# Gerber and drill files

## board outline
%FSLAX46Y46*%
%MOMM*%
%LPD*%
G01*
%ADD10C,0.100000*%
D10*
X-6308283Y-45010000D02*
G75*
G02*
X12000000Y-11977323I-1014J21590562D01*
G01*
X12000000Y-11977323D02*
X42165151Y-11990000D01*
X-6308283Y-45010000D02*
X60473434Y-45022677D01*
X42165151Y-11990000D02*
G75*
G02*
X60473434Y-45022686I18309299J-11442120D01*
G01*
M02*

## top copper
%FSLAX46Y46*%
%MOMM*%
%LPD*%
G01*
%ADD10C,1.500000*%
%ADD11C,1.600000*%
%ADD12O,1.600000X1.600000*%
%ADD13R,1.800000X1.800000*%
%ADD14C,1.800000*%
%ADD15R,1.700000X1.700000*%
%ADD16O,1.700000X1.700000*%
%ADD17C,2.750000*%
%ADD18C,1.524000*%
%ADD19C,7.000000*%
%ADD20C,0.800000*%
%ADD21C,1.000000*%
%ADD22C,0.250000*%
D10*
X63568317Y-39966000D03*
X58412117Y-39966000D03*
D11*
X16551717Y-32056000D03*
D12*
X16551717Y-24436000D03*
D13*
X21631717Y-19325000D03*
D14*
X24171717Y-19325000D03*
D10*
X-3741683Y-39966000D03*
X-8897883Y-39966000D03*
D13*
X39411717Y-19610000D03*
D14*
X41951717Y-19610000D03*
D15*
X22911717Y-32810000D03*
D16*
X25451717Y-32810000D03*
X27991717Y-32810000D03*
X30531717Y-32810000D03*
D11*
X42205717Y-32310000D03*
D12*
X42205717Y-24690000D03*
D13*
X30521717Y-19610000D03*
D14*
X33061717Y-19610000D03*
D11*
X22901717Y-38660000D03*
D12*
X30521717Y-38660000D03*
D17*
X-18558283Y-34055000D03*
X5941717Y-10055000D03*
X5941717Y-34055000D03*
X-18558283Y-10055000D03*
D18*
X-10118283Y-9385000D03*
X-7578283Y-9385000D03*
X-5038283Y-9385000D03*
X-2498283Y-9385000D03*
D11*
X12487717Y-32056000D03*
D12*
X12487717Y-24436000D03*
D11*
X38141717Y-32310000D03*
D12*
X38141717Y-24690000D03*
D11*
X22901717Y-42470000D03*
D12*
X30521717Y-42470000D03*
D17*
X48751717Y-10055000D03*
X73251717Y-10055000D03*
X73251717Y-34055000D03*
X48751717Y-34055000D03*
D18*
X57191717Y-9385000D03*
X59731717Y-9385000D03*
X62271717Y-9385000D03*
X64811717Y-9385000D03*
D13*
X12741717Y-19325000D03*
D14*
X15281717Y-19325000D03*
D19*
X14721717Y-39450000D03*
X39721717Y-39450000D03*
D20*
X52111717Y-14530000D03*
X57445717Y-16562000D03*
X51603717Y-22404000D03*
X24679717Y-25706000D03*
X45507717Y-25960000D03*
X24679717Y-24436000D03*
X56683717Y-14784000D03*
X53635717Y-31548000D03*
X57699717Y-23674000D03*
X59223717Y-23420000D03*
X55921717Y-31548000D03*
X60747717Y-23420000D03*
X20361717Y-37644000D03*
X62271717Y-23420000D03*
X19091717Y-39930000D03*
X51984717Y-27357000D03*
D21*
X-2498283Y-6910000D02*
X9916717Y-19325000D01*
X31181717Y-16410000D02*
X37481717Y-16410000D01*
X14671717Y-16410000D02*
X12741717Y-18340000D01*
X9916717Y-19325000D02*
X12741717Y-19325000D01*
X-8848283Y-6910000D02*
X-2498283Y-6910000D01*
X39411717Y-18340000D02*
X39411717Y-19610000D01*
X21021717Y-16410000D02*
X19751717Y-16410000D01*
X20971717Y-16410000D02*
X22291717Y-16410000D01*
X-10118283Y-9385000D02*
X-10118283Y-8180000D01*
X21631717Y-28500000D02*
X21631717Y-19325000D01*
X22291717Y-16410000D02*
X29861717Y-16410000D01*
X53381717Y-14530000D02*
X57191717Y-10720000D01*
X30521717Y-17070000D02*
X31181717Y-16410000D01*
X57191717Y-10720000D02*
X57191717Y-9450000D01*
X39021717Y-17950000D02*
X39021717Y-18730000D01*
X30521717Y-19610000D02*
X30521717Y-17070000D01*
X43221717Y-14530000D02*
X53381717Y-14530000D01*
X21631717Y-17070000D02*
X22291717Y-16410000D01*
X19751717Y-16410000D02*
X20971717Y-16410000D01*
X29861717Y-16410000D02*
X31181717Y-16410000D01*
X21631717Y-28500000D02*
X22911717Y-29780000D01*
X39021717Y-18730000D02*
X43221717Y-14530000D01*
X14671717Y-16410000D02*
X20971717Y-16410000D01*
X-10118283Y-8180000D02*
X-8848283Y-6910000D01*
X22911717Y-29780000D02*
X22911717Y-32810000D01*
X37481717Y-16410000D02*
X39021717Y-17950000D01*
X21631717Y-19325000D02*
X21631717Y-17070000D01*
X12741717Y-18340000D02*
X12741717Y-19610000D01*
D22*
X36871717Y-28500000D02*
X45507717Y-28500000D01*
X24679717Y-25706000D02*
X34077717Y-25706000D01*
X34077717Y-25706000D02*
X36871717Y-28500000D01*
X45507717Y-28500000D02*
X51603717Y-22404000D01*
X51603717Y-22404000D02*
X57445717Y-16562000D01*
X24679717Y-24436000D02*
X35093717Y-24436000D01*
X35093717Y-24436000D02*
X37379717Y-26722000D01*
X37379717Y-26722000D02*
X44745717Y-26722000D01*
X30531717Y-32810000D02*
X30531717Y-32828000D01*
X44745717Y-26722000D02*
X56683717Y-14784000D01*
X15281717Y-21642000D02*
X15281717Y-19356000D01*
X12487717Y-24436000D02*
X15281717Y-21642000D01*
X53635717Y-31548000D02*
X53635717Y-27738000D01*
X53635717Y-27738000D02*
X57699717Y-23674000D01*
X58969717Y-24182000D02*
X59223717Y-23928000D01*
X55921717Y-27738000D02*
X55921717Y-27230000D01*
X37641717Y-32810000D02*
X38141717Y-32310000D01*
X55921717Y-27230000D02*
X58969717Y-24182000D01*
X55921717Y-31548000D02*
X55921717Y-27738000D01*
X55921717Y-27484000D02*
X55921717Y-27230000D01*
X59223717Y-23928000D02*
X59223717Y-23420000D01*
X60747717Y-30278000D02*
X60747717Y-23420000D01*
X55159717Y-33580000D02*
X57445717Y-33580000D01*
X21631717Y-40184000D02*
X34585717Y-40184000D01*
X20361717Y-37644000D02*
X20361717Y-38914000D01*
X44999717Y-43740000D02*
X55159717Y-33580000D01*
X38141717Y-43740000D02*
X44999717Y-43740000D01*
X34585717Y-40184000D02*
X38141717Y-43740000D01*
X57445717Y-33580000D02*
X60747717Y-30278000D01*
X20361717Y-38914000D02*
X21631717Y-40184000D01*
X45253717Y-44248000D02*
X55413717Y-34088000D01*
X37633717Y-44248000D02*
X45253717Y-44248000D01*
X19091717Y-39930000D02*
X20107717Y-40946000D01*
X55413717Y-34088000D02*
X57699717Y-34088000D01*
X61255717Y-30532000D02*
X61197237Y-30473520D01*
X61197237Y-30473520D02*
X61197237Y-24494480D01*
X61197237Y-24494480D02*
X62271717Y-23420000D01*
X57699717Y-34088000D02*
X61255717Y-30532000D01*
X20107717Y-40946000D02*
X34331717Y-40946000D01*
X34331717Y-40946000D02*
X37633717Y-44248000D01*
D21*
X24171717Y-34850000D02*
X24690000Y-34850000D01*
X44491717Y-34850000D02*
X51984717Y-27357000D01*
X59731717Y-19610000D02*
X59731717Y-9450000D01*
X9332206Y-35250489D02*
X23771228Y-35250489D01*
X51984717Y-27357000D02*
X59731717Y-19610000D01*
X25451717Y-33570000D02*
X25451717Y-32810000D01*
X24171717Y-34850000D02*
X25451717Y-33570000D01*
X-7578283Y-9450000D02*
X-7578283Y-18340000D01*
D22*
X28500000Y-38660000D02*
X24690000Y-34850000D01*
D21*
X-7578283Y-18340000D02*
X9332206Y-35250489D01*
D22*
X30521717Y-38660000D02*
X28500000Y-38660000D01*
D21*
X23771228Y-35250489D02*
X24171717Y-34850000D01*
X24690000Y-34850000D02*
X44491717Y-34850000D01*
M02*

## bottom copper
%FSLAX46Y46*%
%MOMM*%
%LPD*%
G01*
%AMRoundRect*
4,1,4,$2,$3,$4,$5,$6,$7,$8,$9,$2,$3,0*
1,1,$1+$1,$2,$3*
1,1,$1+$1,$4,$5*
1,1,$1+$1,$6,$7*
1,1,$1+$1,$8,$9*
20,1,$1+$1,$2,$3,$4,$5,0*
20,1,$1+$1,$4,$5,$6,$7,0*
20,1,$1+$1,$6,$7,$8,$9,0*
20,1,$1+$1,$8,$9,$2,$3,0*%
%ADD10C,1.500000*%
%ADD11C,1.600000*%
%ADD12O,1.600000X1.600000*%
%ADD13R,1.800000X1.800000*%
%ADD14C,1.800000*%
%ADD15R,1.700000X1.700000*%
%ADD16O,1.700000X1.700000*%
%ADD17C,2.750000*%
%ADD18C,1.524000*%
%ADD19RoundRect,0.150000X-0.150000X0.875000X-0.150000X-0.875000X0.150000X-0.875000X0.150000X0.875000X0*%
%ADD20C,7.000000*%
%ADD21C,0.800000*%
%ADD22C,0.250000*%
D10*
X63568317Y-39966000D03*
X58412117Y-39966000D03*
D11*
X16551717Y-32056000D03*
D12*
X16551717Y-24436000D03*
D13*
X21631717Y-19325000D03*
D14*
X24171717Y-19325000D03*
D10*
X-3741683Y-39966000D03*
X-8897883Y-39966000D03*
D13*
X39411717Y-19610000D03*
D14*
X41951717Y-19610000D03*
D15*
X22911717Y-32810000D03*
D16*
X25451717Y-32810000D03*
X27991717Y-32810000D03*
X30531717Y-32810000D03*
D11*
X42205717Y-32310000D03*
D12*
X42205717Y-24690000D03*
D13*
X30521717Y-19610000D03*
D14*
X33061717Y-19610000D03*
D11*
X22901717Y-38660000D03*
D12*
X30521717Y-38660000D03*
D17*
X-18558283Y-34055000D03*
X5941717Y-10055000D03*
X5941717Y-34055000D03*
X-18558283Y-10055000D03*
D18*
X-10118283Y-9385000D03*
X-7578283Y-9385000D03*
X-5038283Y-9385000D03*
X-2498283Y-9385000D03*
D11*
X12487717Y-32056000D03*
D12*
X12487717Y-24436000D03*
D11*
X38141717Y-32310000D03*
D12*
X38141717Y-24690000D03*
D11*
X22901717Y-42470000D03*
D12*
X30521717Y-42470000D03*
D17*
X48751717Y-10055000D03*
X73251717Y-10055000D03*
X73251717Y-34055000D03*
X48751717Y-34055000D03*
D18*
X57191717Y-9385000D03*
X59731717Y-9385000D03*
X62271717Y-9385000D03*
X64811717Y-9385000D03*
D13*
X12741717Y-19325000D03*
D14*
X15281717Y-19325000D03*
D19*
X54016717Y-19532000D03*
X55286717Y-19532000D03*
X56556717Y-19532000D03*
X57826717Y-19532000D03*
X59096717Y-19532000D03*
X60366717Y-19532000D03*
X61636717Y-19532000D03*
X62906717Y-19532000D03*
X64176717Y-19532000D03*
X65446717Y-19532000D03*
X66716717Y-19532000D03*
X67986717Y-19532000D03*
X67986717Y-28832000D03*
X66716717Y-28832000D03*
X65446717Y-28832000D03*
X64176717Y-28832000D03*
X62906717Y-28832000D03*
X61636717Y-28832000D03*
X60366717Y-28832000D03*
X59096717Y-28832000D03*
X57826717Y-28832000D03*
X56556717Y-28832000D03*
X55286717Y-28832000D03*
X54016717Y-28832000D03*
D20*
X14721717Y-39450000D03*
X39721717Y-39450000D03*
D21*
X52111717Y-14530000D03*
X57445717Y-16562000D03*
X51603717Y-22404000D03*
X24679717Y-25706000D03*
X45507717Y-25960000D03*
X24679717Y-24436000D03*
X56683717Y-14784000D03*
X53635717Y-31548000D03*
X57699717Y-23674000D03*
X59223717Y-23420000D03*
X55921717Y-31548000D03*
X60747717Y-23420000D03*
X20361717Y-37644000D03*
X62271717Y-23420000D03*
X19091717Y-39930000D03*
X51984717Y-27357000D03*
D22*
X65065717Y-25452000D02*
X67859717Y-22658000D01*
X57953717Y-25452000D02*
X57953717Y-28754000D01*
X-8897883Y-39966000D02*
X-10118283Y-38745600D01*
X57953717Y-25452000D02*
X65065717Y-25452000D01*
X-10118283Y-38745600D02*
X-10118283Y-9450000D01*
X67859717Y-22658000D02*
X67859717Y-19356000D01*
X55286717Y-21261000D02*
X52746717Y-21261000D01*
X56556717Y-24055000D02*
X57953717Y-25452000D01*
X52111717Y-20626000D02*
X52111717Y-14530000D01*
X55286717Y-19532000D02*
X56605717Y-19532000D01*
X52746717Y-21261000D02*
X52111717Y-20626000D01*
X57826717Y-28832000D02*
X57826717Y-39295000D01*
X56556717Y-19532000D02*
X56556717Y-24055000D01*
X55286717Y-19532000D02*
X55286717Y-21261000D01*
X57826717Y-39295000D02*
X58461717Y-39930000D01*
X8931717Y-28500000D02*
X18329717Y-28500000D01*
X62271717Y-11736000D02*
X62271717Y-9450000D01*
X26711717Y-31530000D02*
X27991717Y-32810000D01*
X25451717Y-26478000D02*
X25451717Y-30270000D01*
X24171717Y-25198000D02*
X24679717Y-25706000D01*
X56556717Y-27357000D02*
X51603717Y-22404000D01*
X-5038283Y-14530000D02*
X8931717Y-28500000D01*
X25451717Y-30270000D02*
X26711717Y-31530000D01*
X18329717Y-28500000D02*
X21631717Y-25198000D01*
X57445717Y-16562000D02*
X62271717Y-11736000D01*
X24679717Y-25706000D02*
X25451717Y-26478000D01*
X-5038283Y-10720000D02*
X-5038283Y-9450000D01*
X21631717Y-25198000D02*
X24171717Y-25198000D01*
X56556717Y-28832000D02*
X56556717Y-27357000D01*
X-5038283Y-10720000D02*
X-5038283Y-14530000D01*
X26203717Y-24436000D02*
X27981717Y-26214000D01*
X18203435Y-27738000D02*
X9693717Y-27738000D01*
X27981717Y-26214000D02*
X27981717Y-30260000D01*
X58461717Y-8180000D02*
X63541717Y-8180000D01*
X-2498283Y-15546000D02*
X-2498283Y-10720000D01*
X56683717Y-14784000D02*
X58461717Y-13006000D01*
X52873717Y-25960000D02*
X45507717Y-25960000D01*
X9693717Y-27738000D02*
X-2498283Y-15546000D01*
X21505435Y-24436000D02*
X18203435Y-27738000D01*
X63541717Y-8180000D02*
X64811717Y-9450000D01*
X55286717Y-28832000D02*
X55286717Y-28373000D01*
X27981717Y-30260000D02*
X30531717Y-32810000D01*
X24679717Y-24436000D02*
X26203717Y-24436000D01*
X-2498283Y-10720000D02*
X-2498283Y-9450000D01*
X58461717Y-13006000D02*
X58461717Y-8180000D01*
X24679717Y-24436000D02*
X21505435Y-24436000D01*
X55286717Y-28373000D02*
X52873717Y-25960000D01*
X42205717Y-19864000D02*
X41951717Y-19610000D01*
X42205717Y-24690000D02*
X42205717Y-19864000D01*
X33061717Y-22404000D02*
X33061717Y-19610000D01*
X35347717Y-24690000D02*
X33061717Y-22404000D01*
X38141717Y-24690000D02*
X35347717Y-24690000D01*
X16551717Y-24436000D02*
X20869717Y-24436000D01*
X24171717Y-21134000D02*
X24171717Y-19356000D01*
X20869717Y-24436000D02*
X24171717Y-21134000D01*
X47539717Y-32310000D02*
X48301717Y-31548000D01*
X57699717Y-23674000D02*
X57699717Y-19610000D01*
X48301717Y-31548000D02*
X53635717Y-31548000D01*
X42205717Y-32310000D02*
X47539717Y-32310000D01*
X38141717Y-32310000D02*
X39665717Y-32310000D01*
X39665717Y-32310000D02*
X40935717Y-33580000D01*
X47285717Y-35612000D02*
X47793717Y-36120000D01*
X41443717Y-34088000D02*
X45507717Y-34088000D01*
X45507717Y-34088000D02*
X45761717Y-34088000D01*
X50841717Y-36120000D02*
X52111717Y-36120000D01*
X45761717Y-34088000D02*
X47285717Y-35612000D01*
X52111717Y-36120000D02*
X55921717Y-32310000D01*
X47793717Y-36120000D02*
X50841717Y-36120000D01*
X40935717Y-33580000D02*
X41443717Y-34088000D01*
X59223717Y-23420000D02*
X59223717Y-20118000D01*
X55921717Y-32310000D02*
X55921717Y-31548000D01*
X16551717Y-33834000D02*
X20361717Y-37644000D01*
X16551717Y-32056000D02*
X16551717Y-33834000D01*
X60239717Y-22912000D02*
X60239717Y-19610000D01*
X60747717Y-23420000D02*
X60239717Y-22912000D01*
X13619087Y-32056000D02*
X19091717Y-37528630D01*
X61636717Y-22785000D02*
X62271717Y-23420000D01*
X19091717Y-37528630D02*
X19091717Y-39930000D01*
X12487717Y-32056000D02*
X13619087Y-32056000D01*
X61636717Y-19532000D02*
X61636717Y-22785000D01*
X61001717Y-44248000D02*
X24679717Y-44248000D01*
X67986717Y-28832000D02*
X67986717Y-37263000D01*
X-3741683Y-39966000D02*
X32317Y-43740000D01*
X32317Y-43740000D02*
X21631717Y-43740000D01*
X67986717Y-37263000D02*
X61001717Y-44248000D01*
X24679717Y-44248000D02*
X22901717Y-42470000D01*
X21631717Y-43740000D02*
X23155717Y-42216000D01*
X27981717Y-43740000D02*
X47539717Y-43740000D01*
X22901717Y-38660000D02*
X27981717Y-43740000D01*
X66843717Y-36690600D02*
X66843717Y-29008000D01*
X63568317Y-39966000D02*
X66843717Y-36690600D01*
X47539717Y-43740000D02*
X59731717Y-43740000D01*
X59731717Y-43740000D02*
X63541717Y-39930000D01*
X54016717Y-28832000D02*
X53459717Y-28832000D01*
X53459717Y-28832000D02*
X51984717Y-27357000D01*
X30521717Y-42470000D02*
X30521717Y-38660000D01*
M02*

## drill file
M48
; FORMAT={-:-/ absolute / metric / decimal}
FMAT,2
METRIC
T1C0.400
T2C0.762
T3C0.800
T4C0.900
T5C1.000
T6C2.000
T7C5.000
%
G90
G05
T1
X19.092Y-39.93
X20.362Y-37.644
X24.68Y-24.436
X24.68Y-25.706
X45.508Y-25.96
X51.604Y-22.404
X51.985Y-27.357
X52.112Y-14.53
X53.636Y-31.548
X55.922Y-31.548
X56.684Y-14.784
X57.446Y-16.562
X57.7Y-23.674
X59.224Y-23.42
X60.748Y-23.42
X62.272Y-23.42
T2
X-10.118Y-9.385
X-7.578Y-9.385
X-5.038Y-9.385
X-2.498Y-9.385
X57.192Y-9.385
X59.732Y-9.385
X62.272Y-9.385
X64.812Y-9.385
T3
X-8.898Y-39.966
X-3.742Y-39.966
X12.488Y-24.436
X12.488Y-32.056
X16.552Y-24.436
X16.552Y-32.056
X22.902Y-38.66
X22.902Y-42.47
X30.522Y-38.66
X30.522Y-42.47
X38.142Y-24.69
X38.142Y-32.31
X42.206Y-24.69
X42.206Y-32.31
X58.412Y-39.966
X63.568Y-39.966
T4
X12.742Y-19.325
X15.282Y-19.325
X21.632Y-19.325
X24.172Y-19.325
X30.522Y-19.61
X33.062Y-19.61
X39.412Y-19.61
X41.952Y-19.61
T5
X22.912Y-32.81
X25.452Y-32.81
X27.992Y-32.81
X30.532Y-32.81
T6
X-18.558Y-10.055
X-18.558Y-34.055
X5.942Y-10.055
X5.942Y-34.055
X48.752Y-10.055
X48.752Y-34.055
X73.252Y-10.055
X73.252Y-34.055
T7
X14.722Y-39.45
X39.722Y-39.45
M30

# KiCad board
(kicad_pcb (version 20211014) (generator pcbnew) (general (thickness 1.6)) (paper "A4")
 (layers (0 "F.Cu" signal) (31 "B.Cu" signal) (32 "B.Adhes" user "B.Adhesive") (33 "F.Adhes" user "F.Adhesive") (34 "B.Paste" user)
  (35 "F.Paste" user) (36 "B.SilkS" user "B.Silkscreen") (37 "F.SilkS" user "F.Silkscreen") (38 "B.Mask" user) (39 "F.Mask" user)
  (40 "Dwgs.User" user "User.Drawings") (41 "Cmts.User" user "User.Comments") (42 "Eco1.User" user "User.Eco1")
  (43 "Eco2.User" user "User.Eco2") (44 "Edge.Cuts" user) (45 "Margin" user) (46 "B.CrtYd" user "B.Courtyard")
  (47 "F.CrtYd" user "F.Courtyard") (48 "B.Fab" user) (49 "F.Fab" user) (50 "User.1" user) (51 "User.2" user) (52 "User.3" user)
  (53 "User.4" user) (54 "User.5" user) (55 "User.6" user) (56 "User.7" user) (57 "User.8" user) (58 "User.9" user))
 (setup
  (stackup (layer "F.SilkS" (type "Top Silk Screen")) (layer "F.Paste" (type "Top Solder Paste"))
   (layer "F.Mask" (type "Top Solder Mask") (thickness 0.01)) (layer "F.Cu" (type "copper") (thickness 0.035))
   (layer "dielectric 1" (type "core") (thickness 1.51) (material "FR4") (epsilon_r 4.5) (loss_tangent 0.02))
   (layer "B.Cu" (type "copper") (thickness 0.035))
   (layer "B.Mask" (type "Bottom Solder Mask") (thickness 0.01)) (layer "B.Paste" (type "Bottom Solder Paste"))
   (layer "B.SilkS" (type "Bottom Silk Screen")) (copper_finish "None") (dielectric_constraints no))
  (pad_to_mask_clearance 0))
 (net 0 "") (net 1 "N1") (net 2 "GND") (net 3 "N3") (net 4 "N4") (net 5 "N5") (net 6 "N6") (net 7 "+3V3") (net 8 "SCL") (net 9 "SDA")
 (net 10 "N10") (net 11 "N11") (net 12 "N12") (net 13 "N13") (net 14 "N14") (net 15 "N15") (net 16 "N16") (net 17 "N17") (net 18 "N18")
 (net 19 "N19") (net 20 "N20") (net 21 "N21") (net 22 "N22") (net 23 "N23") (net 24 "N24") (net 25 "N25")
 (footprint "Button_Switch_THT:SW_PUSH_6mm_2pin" (layer "F.Cu") (at 57.751717 37.68)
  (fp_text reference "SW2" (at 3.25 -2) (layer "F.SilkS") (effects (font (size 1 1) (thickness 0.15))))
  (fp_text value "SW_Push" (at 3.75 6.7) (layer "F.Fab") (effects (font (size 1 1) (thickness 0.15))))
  (pad "1" thru_hole circle (at 5.8166 2.286 90) (size 1.5 1.5) (drill 0.8) (layers *.Cu *.Mask) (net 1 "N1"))
  (pad "2" thru_hole circle (at 0.6604 2.286 90) (size 1.5 1.5) (drill 0.8) (layers *.Cu *.Mask) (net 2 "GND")))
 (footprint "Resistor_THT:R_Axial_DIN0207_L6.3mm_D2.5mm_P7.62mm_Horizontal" (layer "F.Cu") (at 16.551717 32.056 90)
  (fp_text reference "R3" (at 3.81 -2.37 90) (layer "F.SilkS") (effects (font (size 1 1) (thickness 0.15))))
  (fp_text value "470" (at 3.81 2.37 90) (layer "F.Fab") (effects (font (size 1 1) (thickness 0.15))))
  (pad "1" thru_hole circle (at 0 0 90) (size 1.6 1.6) (drill 0.8) (layers *.Cu *.Mask) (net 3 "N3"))
  (pad "2" thru_hole oval (at 7.62 0 90) (size 1.6 1.6) (drill 0.8) (layers *.Cu *.Mask) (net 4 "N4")))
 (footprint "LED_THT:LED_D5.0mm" (layer "F.Cu") (at 21.631717 19.325)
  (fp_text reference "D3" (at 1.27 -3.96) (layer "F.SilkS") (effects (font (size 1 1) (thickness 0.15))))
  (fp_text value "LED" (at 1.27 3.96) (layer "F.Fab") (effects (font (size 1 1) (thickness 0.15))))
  (pad "1" thru_hole rect (at 0 0) (size 1.8 1.8) (drill 0.9) (layers *.Cu *.Mask) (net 2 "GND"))
  (pad "2" thru_hole circle (at 2.54 0) (size 1.8 1.8) (drill 0.9) (layers *.Cu *.Mask) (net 4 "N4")))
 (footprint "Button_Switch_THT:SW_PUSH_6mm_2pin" (layer "F.Cu") (at -9.558283 37.68)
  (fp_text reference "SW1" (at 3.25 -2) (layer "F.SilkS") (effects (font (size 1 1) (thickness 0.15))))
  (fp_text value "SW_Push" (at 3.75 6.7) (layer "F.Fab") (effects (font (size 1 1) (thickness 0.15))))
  (pad "1" thru_hole circle (at 5.8166 2.286 90) (size 1.5 1.5) (drill 0.8) (layers *.Cu *.Mask) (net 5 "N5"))
  (pad "2" thru_hole circle (at 0.6604 2.286 90) (size 1.5 1.5) (drill 0.8) (layers *.Cu *.Mask) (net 2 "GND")))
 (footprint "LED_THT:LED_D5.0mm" (layer "F.Cu") (at 39.411717 19.61)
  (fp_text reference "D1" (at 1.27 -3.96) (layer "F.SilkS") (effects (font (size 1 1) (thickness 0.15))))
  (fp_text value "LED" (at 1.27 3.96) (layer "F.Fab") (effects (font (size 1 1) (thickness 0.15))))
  (pad "1" thru_hole rect (at 0 0) (size 1.8 1.8) (drill 0.9) (layers *.Cu *.Mask) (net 2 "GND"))
  (pad "2" thru_hole circle (at 2.54 0) (size 1.8 1.8) (drill 0.9) (layers *.Cu *.Mask) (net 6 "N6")))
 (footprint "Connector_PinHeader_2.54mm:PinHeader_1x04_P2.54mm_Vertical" (layer "F.Cu") (at 22.911717 32.81 90)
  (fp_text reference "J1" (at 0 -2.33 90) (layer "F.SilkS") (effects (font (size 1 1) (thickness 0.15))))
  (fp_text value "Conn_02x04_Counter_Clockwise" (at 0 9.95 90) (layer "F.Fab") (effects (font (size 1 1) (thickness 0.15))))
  (pad "1" thru_hole rect (at 0 0 90) (size 1.7 1.7) (drill 1) (layers *.Cu *.Mask) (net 2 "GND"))
  (pad "2" thru_hole oval (at 0 2.54 90) (size 1.7 1.7) (drill 1) (layers *.Cu *.Mask) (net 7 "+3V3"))
  (pad "3" thru_hole oval (at 0 5.08 90) (size 1.7 1.7) (drill 1) (layers *.Cu *.Mask) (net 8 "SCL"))
  (pad "4" thru_hole oval (at 0 7.62 90) (size 1.7 1.7) (drill 1) (layers *.Cu *.Mask) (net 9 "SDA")))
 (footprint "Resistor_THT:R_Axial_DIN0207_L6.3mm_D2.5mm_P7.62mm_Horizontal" (layer "F.Cu") (at 42.205717 32.31 90)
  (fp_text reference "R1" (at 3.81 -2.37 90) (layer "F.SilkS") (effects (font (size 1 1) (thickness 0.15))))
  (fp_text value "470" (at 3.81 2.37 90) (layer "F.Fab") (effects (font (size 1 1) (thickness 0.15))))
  (pad "1" thru_hole circle (at 0 0 90) (size 1.6 1.6) (drill 0.8) (layers *.Cu *.Mask) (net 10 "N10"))
  (pad "2" thru_hole oval (at 7.62 0 90) (size 1.6 1.6) (drill 0.8) (layers *.Cu *.Mask) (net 6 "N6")))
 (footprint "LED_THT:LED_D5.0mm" (layer "F.Cu") (at 30.521717 19.61)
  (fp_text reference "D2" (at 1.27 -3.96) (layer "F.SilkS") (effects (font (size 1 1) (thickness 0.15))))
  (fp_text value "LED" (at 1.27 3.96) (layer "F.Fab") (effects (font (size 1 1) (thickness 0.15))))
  (pad "1" thru_hole rect (at 0 0) (size 1.8 1.8) (drill 0.9) (layers *.Cu *.Mask) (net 2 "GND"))
  (pad "2" thru_hole circle (at 2.54 0) (size 1.8 1.8) (drill 0.9) (layers *.Cu *.Mask) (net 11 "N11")))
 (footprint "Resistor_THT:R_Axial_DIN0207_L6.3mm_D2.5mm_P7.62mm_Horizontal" (layer "F.Cu") (at 22.901717 38.66)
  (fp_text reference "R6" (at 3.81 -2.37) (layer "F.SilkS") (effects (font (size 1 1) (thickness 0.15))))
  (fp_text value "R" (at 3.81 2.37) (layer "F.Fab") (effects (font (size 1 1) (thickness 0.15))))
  (pad "1" thru_hole circle (at 0 0) (size 1.6 1.6) (drill 0.8) (layers *.Cu *.Mask) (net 1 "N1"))
  (pad "2" thru_hole oval (at 7.62 0) (size 1.6 1.6) (drill 0.8) (layers *.Cu *.Mask) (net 7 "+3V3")))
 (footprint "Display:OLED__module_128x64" (layer "F.Cu") (at -6.308283 36.055)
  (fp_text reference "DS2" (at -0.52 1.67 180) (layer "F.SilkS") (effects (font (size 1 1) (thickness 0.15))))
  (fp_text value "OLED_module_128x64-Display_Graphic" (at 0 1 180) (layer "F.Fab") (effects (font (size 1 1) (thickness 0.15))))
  (pad "" thru_hole circle (at -12.25 -2) (size 2.75 2.75) (drill 2) (layers *.Cu *.Mask))
  (pad "" thru_hole circle (at 12.25 -26) (size 2.75 2.75) (drill 2) (layers *.Cu *.Mask))
  (pad "" thru_hole circle (at 12.25 -2) (size 2.75 2.75) (drill 2) (layers *.Cu *.Mask))
  (pad "" thru_hole circle (at -12.25 -26) (size 2.75 2.75) (drill 2) (layers *.Cu *.Mask))
  (pad "1" thru_hole circle (at -3.81 -26.67) (size 1.524 1.524) (drill 0.762) (layers *.Cu *.Mask) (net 2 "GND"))
  (pad "2" thru_hole circle (at -1.27 -26.67) (size 1.524 1.524) (drill 0.762) (layers *.Cu *.Mask) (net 7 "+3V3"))
  (pad "3" thru_hole circle (at 1.27 -26.67) (size 1.524 1.524) (drill 0.762) (layers *.Cu *.Mask) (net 8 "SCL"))
  (pad "4" thru_hole circle (at 3.81 -26.67) (size 1.524 1.524) (drill 0.762) (layers *.Cu *.Mask) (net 9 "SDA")))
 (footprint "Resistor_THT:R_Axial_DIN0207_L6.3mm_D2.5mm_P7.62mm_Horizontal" (layer "F.Cu") (at 12.487717 32.056 90)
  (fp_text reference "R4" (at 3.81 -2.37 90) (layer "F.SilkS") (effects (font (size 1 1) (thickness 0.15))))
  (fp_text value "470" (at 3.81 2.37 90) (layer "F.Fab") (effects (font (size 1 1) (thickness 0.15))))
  (pad "1" thru_hole circle (at 0 0 90) (size 1.6 1.6) (drill 0.8) (layers *.Cu *.Mask) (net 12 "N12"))
  (pad "2" thru_hole oval (at 7.62 0 90) (size 1.6 1.6) (drill 0.8) (layers *.Cu *.Mask) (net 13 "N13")))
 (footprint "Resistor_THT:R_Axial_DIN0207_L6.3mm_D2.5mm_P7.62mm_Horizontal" (layer "F.Cu") (at 38.141717 32.31 90)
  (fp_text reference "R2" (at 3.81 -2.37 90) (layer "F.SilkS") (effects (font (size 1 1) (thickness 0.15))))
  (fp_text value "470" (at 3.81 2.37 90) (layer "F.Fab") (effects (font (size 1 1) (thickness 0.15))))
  (pad "1" thru_hole circle (at 0 0 90) (size 1.6 1.6) (drill 0.8) (layers *.Cu *.Mask) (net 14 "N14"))
  (pad "2" thru_hole oval (at 7.62 0 90) (size 1.6 1.6) (drill 0.8) (layers *.Cu *.Mask) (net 11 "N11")))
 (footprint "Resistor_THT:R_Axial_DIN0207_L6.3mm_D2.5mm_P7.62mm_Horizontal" (layer "F.Cu") (at 22.901717 42.47)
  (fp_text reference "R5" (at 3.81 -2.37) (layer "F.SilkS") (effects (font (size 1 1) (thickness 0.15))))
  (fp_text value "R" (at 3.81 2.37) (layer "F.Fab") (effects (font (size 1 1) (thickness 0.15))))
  (pad "1" thru_hole circle (at 0 0) (size 1.6 1.6) (drill 0.8) (layers *.Cu *.Mask) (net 5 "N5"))
  (pad "2" thru_hole oval (at 7.62 0) (size 1.6 1.6) (drill 0.8) (layers *.Cu *.Mask) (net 7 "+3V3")))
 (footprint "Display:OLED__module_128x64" (layer "F.Cu") (at 61.001717 36.055)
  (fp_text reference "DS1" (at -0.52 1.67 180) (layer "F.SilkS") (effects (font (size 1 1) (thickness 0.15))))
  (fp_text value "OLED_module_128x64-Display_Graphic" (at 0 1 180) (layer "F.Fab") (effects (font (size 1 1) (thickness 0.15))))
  (pad "" thru_hole circle (at -12.25 -26) (size 2.75 2.75) (drill 2) (layers *.Cu *.Mask))
  (pad "" thru_hole circle (at 12.25 -26) (size 2.75 2.75) (drill 2) (layers *.Cu *.Mask))
  (pad "" thru_hole circle (at 12.25 -2) (size 2.75 2.75) (drill 2) (layers *.Cu *.Mask))
  (pad "" thru_hole circle (at -12.25 -2) (size 2.75 2.75) (drill 2) (layers *.Cu *.Mask))
  (pad "1" thru_hole circle (at -3.81 -26.67) (size 1.524 1.524) (drill 0.762) (layers *.Cu *.Mask) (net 2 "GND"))
  (pad "2" thru_hole circle (at -1.27 -26.67) (size 1.524 1.524) (drill 0.762) (layers *.Cu *.Mask) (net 7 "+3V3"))
  (pad "3" thru_hole circle (at 1.27 -26.67) (size 1.524 1.524) (drill 0.762) (layers *.Cu *.Mask) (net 8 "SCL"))
  (pad "4" thru_hole circle (at 3.81 -26.67) (size 1.524 1.524) (drill 0.762) (layers *.Cu *.Mask) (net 9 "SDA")))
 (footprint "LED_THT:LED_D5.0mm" (layer "F.Cu") (at 12.741717 19.325)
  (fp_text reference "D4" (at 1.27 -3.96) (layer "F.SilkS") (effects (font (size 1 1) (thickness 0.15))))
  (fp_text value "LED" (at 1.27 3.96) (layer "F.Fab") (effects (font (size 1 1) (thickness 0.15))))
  (pad "1" thru_hole rect (at 0 0) (size 1.8 1.8) (drill 0.9) (layers *.Cu *.Mask) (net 2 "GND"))
  (pad "2" thru_hole circle (at 2.54 0) (size 1.8 1.8) (drill 0.9) (layers *.Cu *.Mask) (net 13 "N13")))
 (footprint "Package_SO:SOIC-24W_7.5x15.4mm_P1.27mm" (layer "B.Cu") (at 61.001717 24.182 -90)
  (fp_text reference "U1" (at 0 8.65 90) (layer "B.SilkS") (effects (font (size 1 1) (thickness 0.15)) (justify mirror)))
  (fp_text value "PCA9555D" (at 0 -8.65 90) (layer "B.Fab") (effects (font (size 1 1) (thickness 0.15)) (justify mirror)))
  (pad "1" smd roundrect (at -4.65 6.985 270) (size 2.05 0.6) (layers "B.Cu" "B.Paste" "B.Mask") (roundrect_rratio 0.25) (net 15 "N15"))
  (pad "2" smd roundrect (at -4.65 5.715 270) (size 2.05 0.6) (layers "B.Cu" "B.Paste" "B.Mask") (roundrect_rratio 0.25) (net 2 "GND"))
  (pad "3" smd roundrect (at -4.65 4.445 270) (size 2.05 0.6) (layers "B.Cu" "B.Paste" "B.Mask") (roundrect_rratio 0.25) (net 2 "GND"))
  (pad "4" smd roundrect (at -4.65 3.175 270) (size 2.05 0.6) (layers "B.Cu" "B.Paste" "B.Mask") (roundrect_rratio 0.25) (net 10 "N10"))
  (pad "5" smd roundrect (at -4.65 1.905 270) (size 2.05 0.6) (layers "B.Cu" "B.Paste" "B.Mask") (roundrect_rratio 0.25) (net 14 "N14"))
  (pad "6" smd roundrect (at -4.65 0.635 270) (size 2.05 0.6) (layers "B.Cu" "B.Paste" "B.Mask") (roundrect_rratio 0.25) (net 3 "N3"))
  (pad "7" smd roundrect (at -4.65 -0.635 270) (size 2.05 0.6) (layers "B.Cu" "B.Paste" "B.Mask") (roundrect_rratio 0.25) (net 12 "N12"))
  (pad "8" smd roundrect (at -4.65 -1.905 270) (size 2.05 0.6) (layers "B.Cu" "B.Paste" "B.Mask") (roundrect_rratio 0.25) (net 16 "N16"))
  (pad "9" smd roundrect (at -4.65 -3.175 270) (size 2.05 0.6) (layers "B.Cu" "B.Paste" "B.Mask") (roundrect_rratio 0.25) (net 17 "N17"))
  (pad "10" smd roundrect (at -4.65 -4.445 270) (size 2.05 0.6) (layers "B.Cu" "B.Paste" "B.Mask") (roundrect_rratio 0.25) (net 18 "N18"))
  (pad "11" smd roundrect (at -4.65 -5.715 270) (size 2.05 0.6) (layers "B.Cu" "B.Paste" "B.Mask") (roundrect_rratio 0.25) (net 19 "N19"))
  (pad "12" smd roundrect (at -4.65 -6.985 270) (size 2.05 0.6) (layers "B.Cu" "B.Paste" "B.Mask") (roundrect_rratio 0.25) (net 2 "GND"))
  (pad "13" smd roundrect (at 4.65 -6.985 270) (size 2.05 0.6) (layers "B.Cu" "B.Paste" "B.Mask") (roundrect_rratio 0.25) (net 5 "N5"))
  (pad "14" smd roundrect (at 4.65 -5.715 270) (size 2.05 0.6) (layers "B.Cu" "B.Paste" "B.Mask") (roundrect_rratio 0.25) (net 1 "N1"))
  (pad "15" smd roundrect (at 4.65 -4.445 270) (size 2.05 0.6) (layers "B.Cu" "B.Paste" "B.Mask") (roundrect_rratio 0.25) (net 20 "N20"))
  (pad "16" smd roundrect (at 4.65 -3.175 270) (size 2.05 0.6) (layers "B.Cu" "B.Paste" "B.Mask") (roundrect_rratio 0.25) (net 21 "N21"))
  (pad "17" smd roundrect (at 4.65 -1.905 270) (size 2.05 0.6) (layers "B.Cu" "B.Paste" "B.Mask") (roundrect_rratio 0.25) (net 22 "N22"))
  (pad "18" smd roundrect (at 4.65 -0.635 270) (size 2.05 0.6) (layers "B.Cu" "B.Paste" "B.Mask") (roundrect_rratio 0.25) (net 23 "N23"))
  (pad "19" smd roundrect (at 4.65 0.635 270) (size 2.05 0.6) (layers "B.Cu" "B.Paste" "B.Mask") (roundrect_rratio 0.25) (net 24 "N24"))
  (pad "20" smd roundrect (at 4.65 1.905 270) (size 2.05 0.6) (layers "B.Cu" "B.Paste" "B.Mask") (roundrect_rratio 0.25) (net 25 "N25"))
  (pad "21" smd roundrect (at 4.65 3.175 270) (size 2.05 0.6) (layers "B.Cu" "B.Paste" "B.Mask") (roundrect_rratio 0.25) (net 2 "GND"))
  (pad "22" smd roundrect (at 4.65 4.445 270) (size 2.05 0.6) (layers "B.Cu" "B.Paste" "B.Mask") (roundrect_rratio 0.25) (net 8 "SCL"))
  (pad "23" smd roundrect (at 4.65 5.715 270) (size 2.05 0.6) (layers "B.Cu" "B.Paste" "B.Mask") (roundrect_rratio 0.25) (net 9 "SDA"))
  (pad "24" smd roundrect (at 4.65 6.985 270) (size 2.05 0.6) (layers "B.Cu" "B.Paste" "B.Mask") (roundrect_rratio 0.25) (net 7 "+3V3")))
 (gr_arc (start -6.308283 45.01) (mid -25.19332 12.953013) (end 12 11.977323) (layer "Edge.Cuts") (width 0.1))
 (gr_line (start 12 11.977323) (end 42.165151 11.99) (layer "Edge.Cuts") (width 0.1))
 (gr_line (start -6.308283 45.01) (end 60.473434 45.022677) (layer "Edge.Cuts") (width 0.1))
 (gr_arc (start 42.165151 11.99) (mid 79.35847 12.96569) (end 60.473434 45.022677) (layer "Edge.Cuts") (width 0.1))
 (via (at 14.721717 39.45) (size 7) (drill 5) (layers "F.Cu" "B.Cu") (free) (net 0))
 (via (at 39.721717 39.45) (size 7) (drill 5) (layers "F.Cu" "B.Cu") (free) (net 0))
 (segment (start -2.498283 6.91) (end 9.916717 19.325) (width 1) (layer "F.Cu") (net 2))
 (segment (start 31.181717 16.41) (end 37.481717 16.41) (width 1) (layer "F.Cu") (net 2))
 (segment (start 14.671717 16.41) (end 12.741717 18.34) (width 1) (layer "F.Cu") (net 2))
 (segment (start 9.916717 19.325) (end 12.741717 19.325) (width 1) (layer "F.Cu") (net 2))
 (segment (start -8.848283 6.91) (end -2.498283 6.91) (width 1) (layer "F.Cu") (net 2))
 (segment (start 39.411717 18.34) (end 39.411717 19.61) (width 1) (layer "F.Cu") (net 2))
 (segment (start 21.021717 16.41) (end 19.751717 16.41) (width 1) (layer "F.Cu") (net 2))
 (segment (start 20.971717 16.41) (end 22.291717 16.41) (width 1) (layer "F.Cu") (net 2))
 (segment (start -10.118283 9.385) (end -10.118283 8.18) (width 1) (layer "F.Cu") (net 2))
 (segment (start 21.631717 28.5) (end 21.631717 19.325) (width 1) (layer "F.Cu") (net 2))
 (segment (start 22.291717 16.41) (end 29.861717 16.41) (width 1) (layer "F.Cu") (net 2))
 (segment (start 53.381717 14.53) (end 57.191717 10.72) (width 1) (layer "F.Cu") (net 2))
 (segment (start 30.521717 17.07) (end 31.181717 16.41) (width 1) (layer "F.Cu") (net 2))
 (segment (start 57.191717 10.72) (end 57.191717 9.45) (width 1) (layer "F.Cu") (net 2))
 (segment (start 39.021717 17.95) (end 39.021717 18.73) (width 1) (layer "F.Cu") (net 2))
 (segment (start 30.521717 19.61) (end 30.521717 17.07) (width 1) (layer "F.Cu") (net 2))
 (segment (start 43.221717 14.53) (end 53.381717 14.53) (width 1) (layer "F.Cu") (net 2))
 (segment (start 21.631717 17.07) (end 22.291717 16.41) (width 1) (layer "F.Cu") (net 2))
 (segment (start 19.751717 16.41) (end 20.971717 16.41) (width 1) (layer "F.Cu") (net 2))
 (segment (start 29.861717 16.41) (end 31.181717 16.41) (width 1) (layer "F.Cu") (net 2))
 (segment (start 21.631717 28.5) (end 22.911717 29.78) (width 1) (layer "F.Cu") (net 2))
 (segment (start 39.021717 18.73) (end 43.221717 14.53) (width 1) (layer "F.Cu") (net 2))
 (segment (start 14.671717 16.41) (end 20.971717 16.41) (width 1) (layer "F.Cu") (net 2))
 (segment (start -10.118283 8.18) (end -8.848283 6.91) (width 1) (layer "F.Cu") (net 2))
 (segment (start 22.911717 29.78) (end 22.911717 32.81) (width 1) (layer "F.Cu") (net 2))
 (segment (start 37.481717 16.41) (end 39.021717 17.95) (width 1) (layer "F.Cu") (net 2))
 (segment (start 21.631717 19.325) (end 21.631717 17.07) (width 1) (layer "F.Cu") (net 2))
 (segment (start 12.741717 18.34) (end 12.741717 19.61) (width 1) (layer "F.Cu") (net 2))
 (via (at 52.111717 14.53) (size 0.8) (drill 0.4) (layers "F.Cu" "B.Cu") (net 2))
 (segment (start 65.065717 25.452) (end 67.859717 22.658) (width 0.25) (layer "B.Cu") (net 2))
 (segment (start 57.953717 25.452) (end 57.953717 28.754) (width 0.25) (layer "B.Cu") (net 2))
 (segment (start -8.897883 39.966) (end -10.118283 38.7456) (width 0.25) (layer "B.Cu") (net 2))
 (segment (start 57.953717 25.452) (end 65.065717 25.452) (width 0.25) (layer "B.Cu") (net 2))
 (segment (start -10.118283 38.7456) (end -10.118283 9.45) (width 0.25) (layer "B.Cu") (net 2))
 (segment (start 67.859717 22.658) (end 67.859717 19.356) (width 0.25) (layer "B.Cu") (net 2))
 (segment (start 55.286717 21.261) (end 52.746717 21.261) (width 0.25) (layer "B.Cu") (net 2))
 (segment (start 56.556717 24.055) (end 57.953717 25.452) (width 0.25) (layer "B.Cu") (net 2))
 (segment (start 52.111717 20.626) (end 52.111717 14.53) (width 0.25) (layer "B.Cu") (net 2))
 (segment (start 55.286717 19.532) (end 56.605717 19.532) (width 0.25) (layer "B.Cu") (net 2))
 (segment (start 52.746717 21.261) (end 52.111717 20.626) (width 0.25) (layer "B.Cu") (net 2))
 (segment (start 57.826717 28.832) (end 57.826717 39.295) (width 0.25) (layer "B.Cu") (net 2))
 (segment (start 56.556717 19.532) (end 56.556717 24.055) (width 0.25) (layer "B.Cu") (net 2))
 (segment (start 55.286717 19.532) (end 55.286717 21.261) (width 0.25) (layer "B.Cu") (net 2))
 (segment (start 57.826717 39.295) (end 58.461717 39.93) (width 0.25) (layer "B.Cu") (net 2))
 (segment (start 36.871717 28.5) (end 45.507717 28.5) (width 0.25) (layer "F.Cu") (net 8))
 (segment (start 24.679717 25.706) (end 34.077717 25.706) (width 0.25) (layer "F.Cu") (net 8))
 (segment (start 34.077717 25.706) (end 36.871717 28.5) (width 0.25) (layer "F.Cu") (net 8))
 (segment (start 45.507717 28.5) (end 51.603717 22.404) (width 0.25) (layer "F.Cu") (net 8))
 (segment (start 51.603717 22.404) (end 57.445717 16.562) (width 0.25) (layer "F.Cu") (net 8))
 (via (at 57.445717 16.562) (size 0.8) (drill 0.4) (layers "F.Cu" "B.Cu") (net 8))
 (via (at 51.603717 22.404) (size 0.8) (drill 0.4) (layers "F.Cu" "B.Cu") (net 8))
 (via (at 24.679717 25.706) (size 0.8) (drill 0.4) (layers "F.Cu" "B.Cu") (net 8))
 (segment (start 8.931717 28.5) (end 18.329717 28.5) (width 0.25) (layer "B.Cu") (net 8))
 (segment (start 62.271717 11.736) (end 62.271717 9.45) (width 0.25) (layer "B.Cu") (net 8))
 (segment (start 26.711717 31.53) (end 27.991717 32.81) (width 0.25) (layer "B.Cu") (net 8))
 (segment (start 25.451717 26.478) (end 25.451717 30.27) (width 0.25) (layer "B.Cu") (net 8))
 (segment (start 24.171717 25.198) (end 24.679717 25.706) (width 0.25) (layer "B.Cu") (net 8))
 (segment (start 56.556717 27.357) (end 51.603717 22.404) (width 0.25) (layer "B.Cu") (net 8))
 (segment (start -5.038283 14.53) (end 8.931717 28.5) (width 0.25) (layer "B.Cu") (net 8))
 (segment (start 25.451717 30.27) (end 26.711717 31.53) (width 0.25) (layer "B.Cu") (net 8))
 (segment (start 18.329717 28.5) (end 21.631717 25.198) (width 0.25) (layer "B.Cu") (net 8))
 (segment (start 57.445717 16.562) (end 62.271717 11.736) (width 0.25) (layer "B.Cu") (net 8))
 (segment (start 24.679717 25.706) (end 25.451717 26.478) (width 0.25) (layer "B.Cu") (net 8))
 (segment (start -5.038283 10.72) (end -5.038283 9.45) (width 0.25) (layer "B.Cu") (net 8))
 (segment (start 21.631717 25.198) (end 24.171717 25.198) (width 0.25) (layer "B.Cu") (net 8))
 (segment (start 56.556717 28.832) (end 56.556717 27.357) (width 0.25) (layer "B.Cu") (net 8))
 (segment (start -5.038283 10.72) (end -5.038283 14.53) (width 0.25) (layer "B.Cu") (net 8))
 (segment (start 24.679717 24.436) (end 35.093717 24.436) (width 0.25) (layer "F.Cu") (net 9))
 (segment (start 35.093717 24.436) (end 37.379717 26.722) (width 0.25) (layer "F.Cu") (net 9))
 (segment (start 37.379717 26.722) (end 44.745717 26.722) (width 0.25) (layer "F.Cu") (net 9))
 (segment (start 30.531717 32.81) (end 30.531717 32.828) (width 0.25) (layer "F.Cu") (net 9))
 (segment (start 44.745717 26.722) (end 56.683717 14.784) (width 0.25) (layer "F.Cu") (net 9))
 (via (at 45.507717 25.96) (size 0.8) (drill 0.4) (layers "F.Cu" "B.Cu") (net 9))
 (via (at 24.679717 24.436) (size 0.8) (drill 0.4) (layers "F.Cu" "B.Cu") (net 9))
 (via (at 56.683717 14.784) (size 0.8) (drill 0.4) (layers "F.Cu" "B.Cu") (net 9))
 (segment (start 26.203717 24.436) (end 27.981717 26.214) (width 0.25) (layer "B.Cu") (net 9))
 (segment (start 18.203435 27.738) (end 9.693717 27.738) (width 0.25) (layer "B.Cu") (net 9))
 (segment (start 27.981717 26.214) (end 27.981717 30.26) (width 0.25) (layer "B.Cu") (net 9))
 (segment (start 58.461717 8.18) (end 63.541717 8.18) (width 0.25) (layer "B.Cu") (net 9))
 (segment (start -2.498283 15.546) (end -2.498283 10.72) (width 0.25) (layer "B.Cu") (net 9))
 (segment (start 56.683717 14.784) (end 58.461717 13.006) (width 0.25) (layer "B.Cu") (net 9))
 (segment (start 52.873717 25.96) (end 45.507717 25.96) (width 0.25) (layer "B.Cu") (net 9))
 (segment (start 9.693717 27.738) (end -2.498283 15.546) (width 0.25) (layer "B.Cu") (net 9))
 (segment (start 21.505435 24.436) (end 18.203435 27.738) (width 0.25) (layer "B.Cu") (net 9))
 (segment (start 63.541717 8.18) (end 64.811717 9.45) (width 0.25) (layer "B.Cu") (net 9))
 (segment (start 55.286717 28.832) (end 55.286717 28.373) (width 0.25) (layer "B.Cu") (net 9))
 (segment (start 27.981717 30.26) (end 30.531717 32.81) (width 0.25) (layer "B.Cu") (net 9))
 (segment (start 24.679717 24.436) (end 26.203717 24.436) (width 0.25) (layer "B.Cu") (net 9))
 (segment (start -2.498283 10.72) (end -2.498283 9.45) (width 0.25) (layer "B.Cu") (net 9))
 (segment (start 58.461717 13.006) (end 58.461717 8.18) (width 0.25) (layer "B.Cu") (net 9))
 (segment (start 24.679717 24.436) (end 21.505435 24.436) (width 0.25) (layer "B.Cu") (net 9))
 (segment (start 55.286717 28.373) (end 52.873717 25.96) (width 0.25) (layer "B.Cu") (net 9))
 (segment (start 42.205717 19.864) (end 41.951717 19.61) (width 0.25) (layer "B.Cu") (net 6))
 (segment (start 42.205717 24.69) (end 42.205717 19.864) (width 0.25) (layer "B.Cu") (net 6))
 (segment (start 33.061717 22.404) (end 33.061717 19.61) (width 0.25) (layer "B.Cu") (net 11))
 (segment (start 35.347717 24.69) (end 33.061717 22.404) (width 0.25) (layer "B.Cu") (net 11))
 (segment (start 38.141717 24.69) (end 35.347717 24.69) (width 0.25) (layer "B.Cu") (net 11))
 (segment (start 16.551717 24.436) (end 20.869717 24.436) (width 0.25) (layer "B.Cu") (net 4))
 (segment (start 24.171717 21.134) (end 24.171717 19.356) (width 0.25) (layer "B.Cu") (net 4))
 (segment (start 20.869717 24.436) (end 24.171717 21.134) (width 0.25) (layer "B.Cu") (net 4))
 (segment (start 15.281717 21.642) (end 15.281717 19.356) (width 0.25) (layer "F.Cu") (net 13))
 (segment (start 12.487717 24.436) (end 15.281717 21.642) (width 0.25) (layer "F.Cu") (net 13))
 (segment (start 53.635717 31.548) (end 53.635717 27.738) (width 0.25) (layer "F.Cu") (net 10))
 (segment (start 53.635717 27.738) (end 57.699717 23.674) (width 0.25) (layer "F.Cu") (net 10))
 (via (at 53.635717 31.548) (size 0.8) (drill 0.4) (layers "F.Cu" "B.Cu") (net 10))
 (via (at 57.699717 23.674) (size 0.8) (drill 0.4) (layers "F.Cu" "B.Cu") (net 10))
 (segment (start 47.539717 32.31) (end 48.301717 31.548) (width 0.25) (layer "B.Cu") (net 10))
 (segment (start 57.699717 23.674) (end 57.699717 19.61) (width 0.25) (layer "B.Cu") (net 10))
 (segment (start 48.301717 31.548) (end 53.635717 31.548) (width 0.25) (layer "B.Cu") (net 10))
 (segment (start 42.205717 32.31) (end 47.539717 32.31) (width 0.25) (layer "B.Cu") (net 10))
 (segment (start 58.969717 24.182) (end 59.223717 23.928) (width 0.25) (layer "F.Cu") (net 14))
 (segment (start 55.921717 27.738) (end 55.921717 27.23) (width 0.25) (layer "F.Cu") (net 14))
 (segment (start 37.641717 32.81) (end 38.141717 32.31) (width 0.25) (layer "F.Cu") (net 14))
 (segment (start 55.921717 27.23) (end 58.969717 24.182) (width 0.25) (layer "F.Cu") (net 14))
 (segment (start 55.921717 31.548) (end 55.921717 27.738) (width 0.25) (layer "F.Cu") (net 14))
 (segment (start 55.921717 27.484) (end 55.921717 27.23) (width 0.25) (layer "F.Cu") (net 14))
 (segment (start 59.223717 23.928) (end 59.223717 23.42) (width 0.25) (layer "F.Cu") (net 14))
 (via (at 59.223717 23.42) (size 0.8) (drill 0.4) (layers "F.Cu" "B.Cu") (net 14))
 (via (at 55.921717 31.548) (size 0.8) (drill 0.4) (layers "F.Cu" "B.Cu") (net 14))
 (segment (start 38.141717 32.31) (end 39.665717 32.31) (width 0.25) (layer "B.Cu") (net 14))
 (segment (start 39.665717 32.31) (end 40.935717 33.58) (width 0.25) (layer "B.Cu") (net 14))
 (segment (start 47.285717 35.612) (end 47.793717 36.12) (width 0.25) (layer "B.Cu") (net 14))
 (segment (start 41.443717 34.088) (end 45.507717 34.088) (width 0.25) (layer "B.Cu") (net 14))
 (segment (start 45.507717 34.088) (end 45.761717 34.088) (width 0.25) (layer "B.Cu") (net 14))
 (segment (start 50.841717 36.12) (end 52.111717 36.12) (width 0.25) (layer "B.Cu") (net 14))
 (segment (start 45.761717 34.088) (end 47.285717 35.612) (width 0.25) (layer "B.Cu") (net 14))
 (segment (start 52.111717 36.12) (end 55.921717 32.31) (width 0.25) (layer "B.Cu") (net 14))
 (segment (start 47.793717 36.12) (end 50.841717 36.12) (width 0.25) (layer "B.Cu") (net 14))
 (segment (start 40.935717 33.58) (end 41.443717 34.088) (width 0.25) (layer "B.Cu") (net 14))
 (segment (start 59.223717 23.42) (end 59.223717 20.118) (width 0.25) (layer "B.Cu") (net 14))
 (segment (start 55.921717 32.31) (end 55.921717 31.548) (width 0.25) (layer "B.Cu") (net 14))
 (segment (start 60.747717 30.278) (end 60.747717 23.42) (width 0.25) (layer "F.Cu") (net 3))
 (segment (start 55.159717 33.58) (end 57.445717 33.58) (width 0.25) (layer "F.Cu") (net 3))
 (segment (start 21.631717 40.184) (end 34.585717 40.184) (width 0.25) (layer "F.Cu") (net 3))
 (segment (start 20.361717 37.644) (end 20.361717 38.914) (width 0.25) (layer "F.Cu") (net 3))
 (segment (start 44.999717 43.74) (end 55.159717 33.58) (width 0.25) (layer "F.Cu") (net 3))
 (segment (start 38.141717 43.74) (end 44.999717 43.74) (width 0.25) (layer "F.Cu") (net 3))
 (segment (start 34.585717 40.184) (end 38.141717 43.74) (width 0.25) (layer "F.Cu") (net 3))
 (segment (start 57.445717 33.58) (end 60.747717 30.278) (width 0.25) (layer "F.Cu") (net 3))
 (segment (start 20.361717 38.914) (end 21.631717 40.184) (width 0.25) (layer "F.Cu") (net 3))
 (via (at 60.747717 23.42) (size 0.8) (drill 0.4) (layers "F.Cu" "B.Cu") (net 3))
 (via (at 20.361717 37.644) (size 0.8) (drill 0.4) (layers "F.Cu" "B.Cu") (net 3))
 (segment (start 16.551717 33.834) (end 20.361717 37.644) (width 0.25) (layer "B.Cu") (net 3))
 (segment (start 16.551717 32.056) (end 16.551717 33.834) (width 0.25) (layer "B.Cu") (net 3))
 (segment (start 60.239717 22.912) (end 60.239717 19.61) (width 0.25) (layer "B.Cu") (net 3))
 (segment (start 60.747717 23.42) (end 60.239717 22.912) (width 0.25) (layer "B.Cu") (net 3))
 (segment (start 45.253717 44.248) (end 55.413717 34.088) (width 0.25) (layer "F.Cu") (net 12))
 (segment (start 37.633717 44.248) (end 45.253717 44.248) (width 0.25) (layer "F.Cu") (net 12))
 (segment (start 19.091717 39.93) (end 20.107717 40.946) (width 0.25) (layer "F.Cu") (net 12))
 (segment (start 55.413717 34.088) (end 57.699717 34.088) (width 0.25) (layer "F.Cu") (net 12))
 (segment (start 61.255717 30.532) (end 61.197237 30.47352) (width 0.25) (layer "F.Cu") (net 12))
 (segment (start 61.197237 30.47352) (end 61.197237 24.49448) (width 0.25) (layer "F.Cu") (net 12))
 (segment (start 61.197237 24.49448) (end 62.271717 23.42) (width 0.25) (layer "F.Cu") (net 12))
 (segment (start 57.699717 34.088) (end 61.255717 30.532) (width 0.25) (layer "F.Cu") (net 12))
 (segment (start 20.107717 40.946) (end 34.331717 40.946) (width 0.25) (layer "F.Cu") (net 12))
 (segment (start 34.331717 40.946) (end 37.633717 44.248) (width 0.25) (layer "F.Cu") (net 12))
 (via (at 62.271717 23.42) (size 0.8) (drill 0.4) (layers "F.Cu" "B.Cu") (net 12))
 (via (at 19.091717 39.93) (size 0.8) (drill 0.4) (layers "F.Cu" "B.Cu") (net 12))
 (segment (start 13.619087 32.056) (end 19.091717 37.52863) (width 0.25) (layer "B.Cu") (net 12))
 (segment (start 61.636717 22.785) (end 62.271717 23.42) (width 0.25) (layer "B.Cu") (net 12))
 (segment (start 19.091717 37.52863) (end 19.091717 39.93) (width 0.25) (layer "B.Cu") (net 12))
 (segment (start 12.487717 32.056) (end 13.619087 32.056) (width 0.25) (layer "B.Cu") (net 12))
 (segment (start 61.636717 19.532) (end 61.636717 22.785) (width 0.25) (layer "B.Cu") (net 12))
 (segment (start 61.001717 44.248) (end 24.679717 44.248) (width 0.25) (layer "B.Cu") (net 5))
 (segment (start 67.986717 28.832) (end 67.986717 37.263) (width 0.25) (layer "B.Cu") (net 5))
 (segment (start -3.741683 39.966) (end 0.032317 43.74) (width 0.25) (layer "B.Cu") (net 5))
 (segment (start 0.032317 43.74) (end 21.631717 43.74) (width 0.25) (layer "B.Cu") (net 5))
 (segment (start 67.986717 37.263) (end 61.001717 44.248) (width 0.25) (layer "B.Cu") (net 5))
 (segment (start 24.679717 44.248) (end 22.901717 42.47) (width 0.25) (layer "B.Cu") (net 5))
 (segment (start 21.631717 43.74) (end 23.155717 42.216) (width 0.25) (layer "B.Cu") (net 5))
 (segment (start 27.981717 43.74) (end 47.539717 43.74) (width 0.25) (layer "B.Cu") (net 1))
 (segment (start 22.901717 38.66) (end 27.981717 43.74) (width 0.25) (layer "B.Cu") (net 1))
 (segment (start 66.843717 36.6906) (end 66.843717 29.008) (width 0.25) (layer "B.Cu") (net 1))
 (segment (start 63.568317 39.966) (end 66.843717 36.6906) (width 0.25) (layer "B.Cu") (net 1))
 (segment (start 47.539717 43.74) (end 59.731717 43.74) (width 0.25) (layer "B.Cu") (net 1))
 (segment (start 59.731717 43.74) (end 63.541717 39.93) (width 0.25) (layer "B.Cu") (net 1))
 (segment (start 24.171717 34.85) (end 24.69 34.85) (width 1) (layer "F.Cu") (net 7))
 (segment (start 44.491717 34.85) (end 51.984717 27.357) (width 1) (layer "F.Cu") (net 7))
 (segment (start 59.731717 19.61) (end 59.731717 9.45) (width 1) (layer "F.Cu") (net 7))
 (segment (start 9.332206 35.250489) (end 23.771228 35.250489) (width 1) (layer "F.Cu") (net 7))
 (segment (start 51.984717 27.357) (end 59.731717 19.61) (width 1) (layer "F.Cu") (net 7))
 (segment (start 25.451717 33.57) (end 25.451717 32.81) (width 1) (layer "F.Cu") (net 7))
 (segment (start 24.171717 34.85) (end 25.451717 33.57) (width 1) (layer "F.Cu") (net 7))
 (segment (start -7.578283 9.45) (end -7.578283 18.34) (width 1) (layer "F.Cu") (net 7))
 (segment (start 28.5 38.66) (end 24.69 34.85) (width 0.25) (layer "F.Cu") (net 7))
 (segment (start -7.578283 18.34) (end 9.332206 35.250489) (width 1) (layer "F.Cu") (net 7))
 (segment (start 30.521717 38.66) (end 28.5 38.66) (width 0.25) (layer "F.Cu") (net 7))
 (segment (start 23.771228 35.250489) (end 24.171717 34.85) (width 1) (layer "F.Cu") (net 7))
 (segment (start 24.69 34.85) (end 44.491717 34.85) (width 1) (layer "F.Cu") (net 7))
 (via (at 51.984717 27.357) (size 0.8) (drill 0.4) (layers "F.Cu" "B.Cu") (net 7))
 (segment (start 54.016717 28.832) (end 53.459717 28.832) (width 0.25) (layer "B.Cu") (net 7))
 (segment (start 53.459717 28.832) (end 51.984717 27.357) (width 0.25) (layer "B.Cu") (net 7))
 (segment (start 30.521717 42.47) (end 30.521717 38.66) (width 0.25) (layer "B.Cu") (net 7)))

